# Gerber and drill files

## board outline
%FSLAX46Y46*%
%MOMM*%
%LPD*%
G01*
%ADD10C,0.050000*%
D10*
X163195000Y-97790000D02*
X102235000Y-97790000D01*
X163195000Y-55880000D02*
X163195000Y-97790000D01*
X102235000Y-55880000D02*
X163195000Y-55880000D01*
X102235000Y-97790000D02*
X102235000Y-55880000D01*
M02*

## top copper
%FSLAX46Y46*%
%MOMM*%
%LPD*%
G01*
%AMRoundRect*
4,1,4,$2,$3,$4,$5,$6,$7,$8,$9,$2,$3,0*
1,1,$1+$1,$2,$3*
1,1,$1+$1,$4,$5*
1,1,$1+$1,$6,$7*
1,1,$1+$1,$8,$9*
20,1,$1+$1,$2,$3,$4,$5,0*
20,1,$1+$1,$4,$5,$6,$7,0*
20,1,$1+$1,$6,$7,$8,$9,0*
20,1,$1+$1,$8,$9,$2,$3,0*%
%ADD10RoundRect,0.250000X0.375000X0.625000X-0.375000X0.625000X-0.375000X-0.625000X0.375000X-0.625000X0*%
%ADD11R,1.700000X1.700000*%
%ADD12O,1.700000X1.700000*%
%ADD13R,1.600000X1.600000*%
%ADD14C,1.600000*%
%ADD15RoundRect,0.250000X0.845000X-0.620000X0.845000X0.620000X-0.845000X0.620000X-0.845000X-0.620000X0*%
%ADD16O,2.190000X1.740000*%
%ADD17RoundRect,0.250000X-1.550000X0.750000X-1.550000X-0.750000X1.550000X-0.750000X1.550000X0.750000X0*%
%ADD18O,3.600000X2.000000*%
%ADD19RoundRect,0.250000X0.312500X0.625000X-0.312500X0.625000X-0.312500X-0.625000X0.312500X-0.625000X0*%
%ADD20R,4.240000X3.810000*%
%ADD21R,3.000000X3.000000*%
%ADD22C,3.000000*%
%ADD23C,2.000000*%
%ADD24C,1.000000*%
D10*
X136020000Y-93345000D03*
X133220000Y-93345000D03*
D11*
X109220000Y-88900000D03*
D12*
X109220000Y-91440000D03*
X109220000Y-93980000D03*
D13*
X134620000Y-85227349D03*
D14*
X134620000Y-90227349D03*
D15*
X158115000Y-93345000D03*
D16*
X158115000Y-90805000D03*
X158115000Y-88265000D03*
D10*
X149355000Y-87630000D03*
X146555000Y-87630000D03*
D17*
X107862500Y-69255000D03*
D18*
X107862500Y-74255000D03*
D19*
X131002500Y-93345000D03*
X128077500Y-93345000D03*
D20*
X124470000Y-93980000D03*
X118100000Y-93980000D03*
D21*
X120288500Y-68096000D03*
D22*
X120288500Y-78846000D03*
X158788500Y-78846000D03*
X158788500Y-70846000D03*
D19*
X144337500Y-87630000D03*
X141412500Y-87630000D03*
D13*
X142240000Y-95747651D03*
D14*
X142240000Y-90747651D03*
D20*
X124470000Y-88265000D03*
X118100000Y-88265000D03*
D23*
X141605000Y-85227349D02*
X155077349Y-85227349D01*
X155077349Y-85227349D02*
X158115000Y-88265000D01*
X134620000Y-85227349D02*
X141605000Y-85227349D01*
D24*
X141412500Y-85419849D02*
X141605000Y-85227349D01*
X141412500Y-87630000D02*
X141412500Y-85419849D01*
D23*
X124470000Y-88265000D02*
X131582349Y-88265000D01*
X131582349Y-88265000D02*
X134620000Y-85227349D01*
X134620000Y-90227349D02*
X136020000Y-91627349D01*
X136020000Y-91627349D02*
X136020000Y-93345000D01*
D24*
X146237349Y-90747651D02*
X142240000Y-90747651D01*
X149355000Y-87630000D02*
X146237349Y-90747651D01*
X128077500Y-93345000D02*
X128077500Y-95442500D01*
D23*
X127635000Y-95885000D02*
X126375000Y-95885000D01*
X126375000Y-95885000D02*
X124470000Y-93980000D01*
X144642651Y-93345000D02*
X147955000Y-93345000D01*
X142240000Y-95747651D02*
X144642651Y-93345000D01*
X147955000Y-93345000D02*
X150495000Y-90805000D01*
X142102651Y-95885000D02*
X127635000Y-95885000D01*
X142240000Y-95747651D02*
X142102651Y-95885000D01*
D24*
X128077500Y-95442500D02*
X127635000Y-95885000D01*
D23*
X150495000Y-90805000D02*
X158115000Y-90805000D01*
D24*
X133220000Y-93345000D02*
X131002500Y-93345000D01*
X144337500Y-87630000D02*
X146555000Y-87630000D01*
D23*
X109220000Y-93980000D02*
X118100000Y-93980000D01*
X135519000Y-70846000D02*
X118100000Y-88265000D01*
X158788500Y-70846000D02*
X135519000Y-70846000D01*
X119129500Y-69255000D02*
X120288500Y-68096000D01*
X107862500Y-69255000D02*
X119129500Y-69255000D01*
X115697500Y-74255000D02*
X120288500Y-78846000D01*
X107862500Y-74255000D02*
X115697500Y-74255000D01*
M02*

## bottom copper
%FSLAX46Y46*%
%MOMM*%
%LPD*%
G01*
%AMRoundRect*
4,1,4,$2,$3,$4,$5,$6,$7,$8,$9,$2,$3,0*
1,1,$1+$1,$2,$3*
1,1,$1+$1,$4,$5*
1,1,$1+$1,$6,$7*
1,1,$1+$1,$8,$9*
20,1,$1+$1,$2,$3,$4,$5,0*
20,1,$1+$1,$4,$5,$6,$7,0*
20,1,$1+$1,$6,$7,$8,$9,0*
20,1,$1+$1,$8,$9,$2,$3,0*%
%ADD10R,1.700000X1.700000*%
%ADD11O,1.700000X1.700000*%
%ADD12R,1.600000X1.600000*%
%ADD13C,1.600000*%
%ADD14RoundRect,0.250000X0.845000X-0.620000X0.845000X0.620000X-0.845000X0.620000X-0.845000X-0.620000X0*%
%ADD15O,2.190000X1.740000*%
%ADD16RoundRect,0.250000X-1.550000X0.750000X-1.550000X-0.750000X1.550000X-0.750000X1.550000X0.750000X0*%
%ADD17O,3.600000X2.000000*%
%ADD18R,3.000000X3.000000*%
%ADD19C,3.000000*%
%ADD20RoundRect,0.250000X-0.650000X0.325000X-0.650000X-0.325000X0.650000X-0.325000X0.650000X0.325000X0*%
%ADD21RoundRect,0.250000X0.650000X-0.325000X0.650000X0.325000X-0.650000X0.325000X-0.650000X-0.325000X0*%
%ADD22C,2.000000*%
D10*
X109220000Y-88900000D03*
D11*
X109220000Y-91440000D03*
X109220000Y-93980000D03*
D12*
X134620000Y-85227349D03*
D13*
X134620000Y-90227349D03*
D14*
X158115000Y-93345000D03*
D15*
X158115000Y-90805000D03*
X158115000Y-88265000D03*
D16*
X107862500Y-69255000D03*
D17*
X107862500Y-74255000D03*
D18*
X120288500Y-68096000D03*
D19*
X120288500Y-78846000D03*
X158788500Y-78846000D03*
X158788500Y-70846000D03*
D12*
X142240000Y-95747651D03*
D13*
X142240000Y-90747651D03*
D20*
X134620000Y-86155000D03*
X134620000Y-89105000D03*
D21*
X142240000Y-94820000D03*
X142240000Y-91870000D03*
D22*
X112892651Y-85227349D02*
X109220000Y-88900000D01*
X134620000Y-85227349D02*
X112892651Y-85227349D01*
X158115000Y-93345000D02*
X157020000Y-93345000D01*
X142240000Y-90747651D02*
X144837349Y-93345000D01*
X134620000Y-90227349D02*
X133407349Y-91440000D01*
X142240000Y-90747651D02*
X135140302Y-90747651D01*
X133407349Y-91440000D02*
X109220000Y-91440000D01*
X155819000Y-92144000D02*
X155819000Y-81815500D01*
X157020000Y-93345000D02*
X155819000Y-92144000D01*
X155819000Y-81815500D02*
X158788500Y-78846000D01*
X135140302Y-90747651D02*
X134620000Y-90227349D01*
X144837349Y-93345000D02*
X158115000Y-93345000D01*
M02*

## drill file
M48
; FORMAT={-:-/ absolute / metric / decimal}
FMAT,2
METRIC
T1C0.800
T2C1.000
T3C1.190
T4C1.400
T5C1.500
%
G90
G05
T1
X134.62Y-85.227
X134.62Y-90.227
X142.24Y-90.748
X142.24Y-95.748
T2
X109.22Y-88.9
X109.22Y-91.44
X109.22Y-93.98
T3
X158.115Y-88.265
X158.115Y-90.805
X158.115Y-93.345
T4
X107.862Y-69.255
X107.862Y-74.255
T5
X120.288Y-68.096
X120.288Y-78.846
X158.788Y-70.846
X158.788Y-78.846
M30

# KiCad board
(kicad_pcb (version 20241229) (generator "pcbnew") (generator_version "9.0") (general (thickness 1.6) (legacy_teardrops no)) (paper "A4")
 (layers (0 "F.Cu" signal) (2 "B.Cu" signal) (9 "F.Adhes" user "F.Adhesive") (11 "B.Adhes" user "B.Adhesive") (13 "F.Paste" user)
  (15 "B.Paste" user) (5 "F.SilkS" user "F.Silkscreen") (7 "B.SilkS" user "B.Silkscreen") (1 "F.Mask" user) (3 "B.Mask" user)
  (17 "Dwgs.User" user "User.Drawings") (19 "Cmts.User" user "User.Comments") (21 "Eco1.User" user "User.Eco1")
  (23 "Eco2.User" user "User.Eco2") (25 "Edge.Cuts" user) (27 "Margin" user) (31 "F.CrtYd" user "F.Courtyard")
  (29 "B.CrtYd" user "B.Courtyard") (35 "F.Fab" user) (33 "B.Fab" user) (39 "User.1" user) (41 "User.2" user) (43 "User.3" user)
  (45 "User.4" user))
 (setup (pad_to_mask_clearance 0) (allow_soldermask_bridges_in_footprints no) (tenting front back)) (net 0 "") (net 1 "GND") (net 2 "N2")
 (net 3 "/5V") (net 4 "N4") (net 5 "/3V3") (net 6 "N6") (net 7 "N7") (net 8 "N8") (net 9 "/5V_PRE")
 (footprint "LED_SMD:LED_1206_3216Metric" (layer "F.Cu") (at 134.62 93.345 180)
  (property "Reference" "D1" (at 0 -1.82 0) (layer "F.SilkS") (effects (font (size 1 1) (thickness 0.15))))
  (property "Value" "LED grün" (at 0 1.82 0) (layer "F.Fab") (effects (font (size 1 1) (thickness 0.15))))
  (pad "1" smd roundrect (at -1.4 0 180) (size 1.25 1.75) (layers "F.Cu" "F.Mask" "F.Paste") (roundrect_rratio 0.2) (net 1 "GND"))
  (pad "2" smd roundrect (at 1.4 0 180) (size 1.25 1.75) (layers "F.Cu" "F.Mask" "F.Paste") (roundrect_rratio 0.2) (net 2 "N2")))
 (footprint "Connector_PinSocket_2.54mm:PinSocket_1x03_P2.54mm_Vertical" (layer "F.Cu") (at 109.22 88.9)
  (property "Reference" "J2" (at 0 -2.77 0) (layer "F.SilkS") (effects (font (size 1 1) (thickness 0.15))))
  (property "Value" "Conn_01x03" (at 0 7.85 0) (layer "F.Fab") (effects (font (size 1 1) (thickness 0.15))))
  (pad "1" thru_hole rect (at 0 0) (size 1.7 1.7) (drill 1) (layers "*.Cu" "*.Mask") (remove_unused_layers no) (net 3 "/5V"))
  (pad "2" thru_hole oval (at 0 2.54) (size 1.7 1.7) (drill 1) (layers "*.Cu" "*.Mask") (remove_unused_layers no) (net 1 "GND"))
  (pad "3" thru_hole oval (at 0 5.08) (size 1.7 1.7) (drill 1) (layers "*.Cu" "*.Mask") (remove_unused_layers no) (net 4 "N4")))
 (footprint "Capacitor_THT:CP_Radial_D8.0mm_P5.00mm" (layer "F.Cu") (at 134.62 85.227349 -90)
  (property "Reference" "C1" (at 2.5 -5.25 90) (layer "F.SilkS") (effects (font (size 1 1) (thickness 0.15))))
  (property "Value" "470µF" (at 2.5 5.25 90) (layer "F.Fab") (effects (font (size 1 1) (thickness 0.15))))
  (pad "1" thru_hole rect (at 0 0 270) (size 1.6 1.6) (drill 0.8) (layers "*.Cu" "*.Mask") (remove_unused_layers no) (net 3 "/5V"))
  (pad "2" thru_hole circle (at 5 0 270) (size 1.6 1.6) (drill 0.8) (layers "*.Cu" "*.Mask") (remove_unused_layers no) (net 1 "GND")))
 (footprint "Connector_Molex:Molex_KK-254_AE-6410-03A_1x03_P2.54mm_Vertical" (layer "F.Cu") (at 158.115 93.345 90)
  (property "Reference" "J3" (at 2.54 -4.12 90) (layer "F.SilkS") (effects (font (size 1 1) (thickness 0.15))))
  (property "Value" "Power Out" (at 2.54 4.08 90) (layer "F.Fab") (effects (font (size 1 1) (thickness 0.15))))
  (pad "1" thru_hole roundrect (at 0 0 90) (size 1.74 2.19) (drill 1.19) (layers "*.Cu" "*.Mask") (remove_unused_layers no)
   (roundrect_rratio 0.143678) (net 1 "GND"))
  (pad "2" thru_hole oval (at 2.54 0 90) (size 1.74 2.19) (drill 1.19) (layers "*.Cu" "*.Mask") (remove_unused_layers no) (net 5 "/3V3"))
  (pad "3" thru_hole oval (at 5.08 0 90) (size 1.74 2.19) (drill 1.19) (layers "*.Cu" "*.Mask") (remove_unused_layers no) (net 3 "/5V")))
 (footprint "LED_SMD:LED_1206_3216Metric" (layer "F.Cu") (at 147.955 87.63 180)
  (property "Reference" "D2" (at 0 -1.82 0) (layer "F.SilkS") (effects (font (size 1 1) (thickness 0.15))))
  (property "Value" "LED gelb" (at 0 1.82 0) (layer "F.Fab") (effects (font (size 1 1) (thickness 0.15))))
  (pad "1" smd roundrect (at -1.4 0 180) (size 1.25 1.75) (layers "F.Cu" "F.Mask" "F.Paste") (roundrect_rratio 0.2) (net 1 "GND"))
  (pad "2" smd roundrect (at 1.4 0 180) (size 1.25 1.75) (layers "F.Cu" "F.Mask" "F.Paste") (roundrect_rratio 0.2) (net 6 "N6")))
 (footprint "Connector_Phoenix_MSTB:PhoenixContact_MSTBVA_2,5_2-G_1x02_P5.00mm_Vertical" (layer "F.Cu") (at 107.8625 69.255 -90)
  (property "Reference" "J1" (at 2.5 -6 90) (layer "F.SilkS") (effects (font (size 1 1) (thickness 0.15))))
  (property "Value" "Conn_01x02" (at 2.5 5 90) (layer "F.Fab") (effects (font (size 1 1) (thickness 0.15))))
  (pad "1" thru_hole roundrect (at 0 0 270) (size 2 3.6) (drill 1.4) (layers "*.Cu" "*.Mask") (remove_unused_layers no)
   (roundrect_rratio 0.125) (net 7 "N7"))
  (pad "2" thru_hole oval (at 5 0 270) (size 2 3.6) (drill 1.4) (layers "*.Cu" "*.Mask") (remove_unused_layers no) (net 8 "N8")))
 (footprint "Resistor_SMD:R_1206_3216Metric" (layer "F.Cu") (at 129.54 93.345 180)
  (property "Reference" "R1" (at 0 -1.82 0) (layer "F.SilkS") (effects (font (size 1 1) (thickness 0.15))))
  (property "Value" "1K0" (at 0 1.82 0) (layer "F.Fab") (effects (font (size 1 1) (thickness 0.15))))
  (pad "1" smd roundrect (at -1.4625 0 180) (size 1.125 1.75) (layers "F.Cu" "F.Mask" "F.Paste") (roundrect_rratio 0.222222) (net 2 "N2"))
  (pad "2" smd roundrect (at 1.4625 0 180) (size 1.125 1.75) (layers "F.Cu" "F.Mask" "F.Paste") (roundrect_rratio 0.222222) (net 5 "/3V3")))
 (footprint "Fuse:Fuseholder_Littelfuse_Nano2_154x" (layer "F.Cu") (at 121.285 93.98 180)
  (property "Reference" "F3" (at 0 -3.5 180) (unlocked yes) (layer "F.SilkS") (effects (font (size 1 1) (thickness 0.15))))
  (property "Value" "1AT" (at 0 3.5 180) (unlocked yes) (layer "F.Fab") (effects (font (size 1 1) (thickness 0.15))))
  (pad "1" smd rect (at -3.185 0 180) (size 4.24 3.81) (layers "F.Cu" "F.Mask" "F.Paste") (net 5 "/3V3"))
  (pad "2" smd rect (at 3.185 0 180) (size 4.24 3.81) (layers "F.Cu" "F.Mask" "F.Paste") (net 4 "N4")))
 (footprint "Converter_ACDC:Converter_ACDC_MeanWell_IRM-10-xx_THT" (layer "F.Cu") (at 120.2885 68.096)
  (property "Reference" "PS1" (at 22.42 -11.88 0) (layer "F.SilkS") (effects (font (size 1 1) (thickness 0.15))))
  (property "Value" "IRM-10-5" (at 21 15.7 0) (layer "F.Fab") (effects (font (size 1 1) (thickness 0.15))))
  (pad "1" thru_hole rect (at 0 0) (size 3 3) (drill 1.5) (layers "*.Cu" "*.Mask") (remove_unused_layers no) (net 7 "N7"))
  (pad "2" thru_hole circle (at 0 10.75) (size 3 3) (drill 1.5) (layers "*.Cu" "*.Mask") (remove_unused_layers no) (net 8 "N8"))
  (pad "3" thru_hole circle (at 38.5 10.75) (size 3 3) (drill 1.5) (layers "*.Cu" "*.Mask") (remove_unused_layers no) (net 1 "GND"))
  (pad "4" thru_hole circle (at 38.5 2.75) (size 3 3) (drill 1.5) (layers "*.Cu" "*.Mask") (remove_unused_layers no) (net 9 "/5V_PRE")))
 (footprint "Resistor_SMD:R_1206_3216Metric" (layer "F.Cu") (at 142.875 87.63 180)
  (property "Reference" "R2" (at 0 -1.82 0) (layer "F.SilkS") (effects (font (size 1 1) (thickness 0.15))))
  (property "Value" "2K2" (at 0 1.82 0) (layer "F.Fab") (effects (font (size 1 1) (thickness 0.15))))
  (pad "1" smd roundrect (at -1.4625 0 180) (size 1.125 1.75) (layers "F.Cu" "F.Mask" "F.Paste") (roundrect_rratio 0.222222) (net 6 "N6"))
  (pad "2" smd roundrect (at 1.4625 0 180) (size 1.125 1.75) (layers "F.Cu" "F.Mask" "F.Paste") (roundrect_rratio 0.222222) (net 3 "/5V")))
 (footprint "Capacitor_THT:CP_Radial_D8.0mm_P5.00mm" (layer "F.Cu") (at 142.24 95.747651 90)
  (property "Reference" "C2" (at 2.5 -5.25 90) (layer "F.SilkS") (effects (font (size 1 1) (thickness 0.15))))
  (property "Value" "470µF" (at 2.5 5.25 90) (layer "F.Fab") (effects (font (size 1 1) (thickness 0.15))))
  (pad "1" thru_hole rect (at 0 0 90) (size 1.6 1.6) (drill 0.8) (layers "*.Cu" "*.Mask") (remove_unused_layers no) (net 5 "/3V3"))
  (pad "2" thru_hole circle (at 5 0 90) (size 1.6 1.6) (drill 0.8) (layers "*.Cu" "*.Mask") (remove_unused_layers no) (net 1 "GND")))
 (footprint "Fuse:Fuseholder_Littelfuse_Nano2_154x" (layer "F.Cu") (at 121.285 88.265 180)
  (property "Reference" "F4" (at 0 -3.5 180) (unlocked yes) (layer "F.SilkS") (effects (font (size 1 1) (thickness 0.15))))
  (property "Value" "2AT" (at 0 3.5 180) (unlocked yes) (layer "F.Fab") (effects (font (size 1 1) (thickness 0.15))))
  (pad "1" smd rect (at -3.185 0 180) (size 4.24 3.81) (layers "F.Cu" "F.Mask" "F.Paste") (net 3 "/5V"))
  (pad "2" smd rect (at 3.185 0 180) (size 4.24 3.81) (layers "F.Cu" "F.Mask" "F.Paste") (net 9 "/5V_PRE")))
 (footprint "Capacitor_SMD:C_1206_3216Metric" (layer "B.Cu") (at 134.62 87.63 -90)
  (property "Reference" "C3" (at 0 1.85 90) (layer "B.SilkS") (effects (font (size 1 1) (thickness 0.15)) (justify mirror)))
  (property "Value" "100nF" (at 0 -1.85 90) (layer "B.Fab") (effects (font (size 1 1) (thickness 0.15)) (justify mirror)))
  (pad "1" smd roundrect (at -1.475 0 270) (size 1.15 1.8) (layers "B.Cu" "B.Mask" "B.Paste") (roundrect_rratio 0.217391) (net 3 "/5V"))
  (pad "2" smd roundrect (at 1.475 0 270) (size 1.15 1.8) (layers "B.Cu" "B.Mask" "B.Paste") (roundrect_rratio 0.217391) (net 1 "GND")))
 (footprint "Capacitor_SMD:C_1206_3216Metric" (layer "B.Cu") (at 142.24 93.345 90)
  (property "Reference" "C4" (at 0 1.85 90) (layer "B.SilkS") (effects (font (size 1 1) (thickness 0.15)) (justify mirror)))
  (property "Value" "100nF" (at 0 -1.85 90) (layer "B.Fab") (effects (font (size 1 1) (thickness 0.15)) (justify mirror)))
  (pad "1" smd roundrect (at -1.475 0 90) (size 1.15 1.8) (layers "B.Cu" "B.Mask" "B.Paste") (roundrect_rratio 0.217391) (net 5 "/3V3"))
  (pad "2" smd roundrect (at 1.475 0 90) (size 1.15 1.8) (layers "B.Cu" "B.Mask" "B.Paste") (roundrect_rratio 0.217391) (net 1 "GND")))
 (gr_line (start 163.195 97.79) (end 102.235 97.79) (stroke (width 0.05) (type default)) (layer "Edge.Cuts"))
 (gr_line (start 163.195 55.88) (end 163.195 97.79) (stroke (width 0.05) (type default)) (layer "Edge.Cuts"))
 (gr_line (start 102.235 55.88) (end 163.195 55.88) (stroke (width 0.05) (type default)) (layer "Edge.Cuts"))
 (gr_line (start 102.235 97.79) (end 102.235 55.88) (stroke (width 0.05) (type default)) (layer "Edge.Cuts"))
 (segment (start 141.605 85.227349) (end 155.077349 85.227349) (width 2) (layer "F.Cu") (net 3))
 (segment (start 155.077349 85.227349) (end 158.115 88.265) (width 2) (layer "F.Cu") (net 3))
 (segment (start 134.62 85.227349) (end 141.605 85.227349) (width 2) (layer "F.Cu") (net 3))
 (segment (start 141.4125 85.419849) (end 141.605 85.227349) (width 1) (layer "F.Cu") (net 3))
 (segment (start 141.4125 87.63) (end 141.4125 85.419849) (width 1) (layer "F.Cu") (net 3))
 (segment (start 124.47 88.265) (end 131.582349 88.265) (width 2) (layer "F.Cu") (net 3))
 (segment (start 131.582349 88.265) (end 134.62 85.227349) (width 2) (layer "F.Cu") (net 3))
 (segment (start 112.892651 85.227349) (end 109.22 88.9) (width 2) (layer "B.Cu") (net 3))
 (segment (start 134.62 85.227349) (end 112.892651 85.227349) (width 2) (layer "B.Cu") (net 3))
 (segment (start 134.62 90.227349) (end 136.02 91.627349) (width 2) (layer "F.Cu") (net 1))
 (segment (start 136.02 91.627349) (end 136.02 93.345) (width 2) (layer "F.Cu") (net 1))
 (segment (start 146.237349 90.747651) (end 142.24 90.747651) (width 1) (layer "F.Cu") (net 1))
 (segment (start 149.355 87.63) (end 146.237349 90.747651) (width 1) (layer "F.Cu") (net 1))
 (segment (start 158.115 93.345) (end 157.02 93.345) (width 2) (layer "B.Cu") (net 1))
 (segment (start 142.24 90.747651) (end 144.837349 93.345) (width 2) (layer "B.Cu") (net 1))
 (segment (start 134.62 90.227349) (end 133.407349 91.44) (width 2) (layer "B.Cu") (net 1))
 (segment (start 142.24 90.747651) (end 135.140302 90.747651) (width 2) (layer "B.Cu") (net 1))
 (segment (start 133.407349 91.44) (end 109.22 91.44) (width 2) (layer "B.Cu") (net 1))
 (segment (start 155.819 92.144) (end 155.819 81.8155) (width 2) (layer "B.Cu") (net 1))
 (segment (start 157.02 93.345) (end 155.819 92.144) (width 2) (layer "B.Cu") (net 1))
 (segment (start 155.819 81.8155) (end 158.7885 78.846) (width 2) (layer "B.Cu") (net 1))
 (segment (start 135.140302 90.747651) (end 134.62 90.227349) (width 2) (layer "B.Cu") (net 1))
 (segment (start 144.837349 93.345) (end 158.115 93.345) (width 2) (layer "B.Cu") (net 1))
 (segment (start 128.0775 93.345) (end 128.0775 95.4425) (width 1) (layer "F.Cu") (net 5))
 (segment (start 127.635 95.885) (end 126.375 95.885) (width 2) (layer "F.Cu") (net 5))
 (segment (start 126.375 95.885) (end 124.47 93.98) (width 2) (layer "F.Cu") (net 5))
 (segment (start 144.642651 93.345) (end 147.955 93.345) (width 2) (layer "F.Cu") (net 5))
 (segment (start 142.24 95.747651) (end 144.642651 93.345) (width 2) (layer "F.Cu") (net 5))
 (segment (start 147.955 93.345) (end 150.495 90.805) (width 2) (layer "F.Cu") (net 5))
 (segment (start 142.102651 95.885) (end 127.635 95.885) (width 2) (layer "F.Cu") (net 5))
 (segment (start 142.24 95.747651) (end 142.102651 95.885) (width 2) (layer "F.Cu") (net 5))
 (segment (start 128.0775 95.4425) (end 127.635 95.885) (width 1) (layer "F.Cu") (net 5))
 (segment (start 150.495 90.805) (end 158.115 90.805) (width 2) (layer "F.Cu") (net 5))
 (segment (start 133.22 93.345) (end 131.0025 93.345) (width 1) (layer "F.Cu") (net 2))
 (segment (start 144.3375 87.63) (end 146.555 87.63) (width 1) (layer "F.Cu") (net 6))
 (segment (start 109.22 93.98) (end 118.1 93.98) (width 2) (layer "F.Cu") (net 4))
 (segment (start 135.519 70.846) (end 118.1 88.265) (width 2) (layer "F.Cu") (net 9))
 (segment (start 158.7885 70.846) (end 135.519 70.846) (width 2) (layer "F.Cu") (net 9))
 (segment (start 119.1295 69.255) (end 120.2885 68.096) (width 2) (layer "F.Cu") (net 7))
 (segment (start 107.8625 69.255) (end 119.1295 69.255) (width 2) (layer "F.Cu") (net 7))
 (segment (start 115.6975 74.255) (end 120.2885 78.846) (width 2) (layer "F.Cu") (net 8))
 (segment (start 107.8625 74.255) (end 115.6975 74.255) (width 2) (layer "F.Cu") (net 8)))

